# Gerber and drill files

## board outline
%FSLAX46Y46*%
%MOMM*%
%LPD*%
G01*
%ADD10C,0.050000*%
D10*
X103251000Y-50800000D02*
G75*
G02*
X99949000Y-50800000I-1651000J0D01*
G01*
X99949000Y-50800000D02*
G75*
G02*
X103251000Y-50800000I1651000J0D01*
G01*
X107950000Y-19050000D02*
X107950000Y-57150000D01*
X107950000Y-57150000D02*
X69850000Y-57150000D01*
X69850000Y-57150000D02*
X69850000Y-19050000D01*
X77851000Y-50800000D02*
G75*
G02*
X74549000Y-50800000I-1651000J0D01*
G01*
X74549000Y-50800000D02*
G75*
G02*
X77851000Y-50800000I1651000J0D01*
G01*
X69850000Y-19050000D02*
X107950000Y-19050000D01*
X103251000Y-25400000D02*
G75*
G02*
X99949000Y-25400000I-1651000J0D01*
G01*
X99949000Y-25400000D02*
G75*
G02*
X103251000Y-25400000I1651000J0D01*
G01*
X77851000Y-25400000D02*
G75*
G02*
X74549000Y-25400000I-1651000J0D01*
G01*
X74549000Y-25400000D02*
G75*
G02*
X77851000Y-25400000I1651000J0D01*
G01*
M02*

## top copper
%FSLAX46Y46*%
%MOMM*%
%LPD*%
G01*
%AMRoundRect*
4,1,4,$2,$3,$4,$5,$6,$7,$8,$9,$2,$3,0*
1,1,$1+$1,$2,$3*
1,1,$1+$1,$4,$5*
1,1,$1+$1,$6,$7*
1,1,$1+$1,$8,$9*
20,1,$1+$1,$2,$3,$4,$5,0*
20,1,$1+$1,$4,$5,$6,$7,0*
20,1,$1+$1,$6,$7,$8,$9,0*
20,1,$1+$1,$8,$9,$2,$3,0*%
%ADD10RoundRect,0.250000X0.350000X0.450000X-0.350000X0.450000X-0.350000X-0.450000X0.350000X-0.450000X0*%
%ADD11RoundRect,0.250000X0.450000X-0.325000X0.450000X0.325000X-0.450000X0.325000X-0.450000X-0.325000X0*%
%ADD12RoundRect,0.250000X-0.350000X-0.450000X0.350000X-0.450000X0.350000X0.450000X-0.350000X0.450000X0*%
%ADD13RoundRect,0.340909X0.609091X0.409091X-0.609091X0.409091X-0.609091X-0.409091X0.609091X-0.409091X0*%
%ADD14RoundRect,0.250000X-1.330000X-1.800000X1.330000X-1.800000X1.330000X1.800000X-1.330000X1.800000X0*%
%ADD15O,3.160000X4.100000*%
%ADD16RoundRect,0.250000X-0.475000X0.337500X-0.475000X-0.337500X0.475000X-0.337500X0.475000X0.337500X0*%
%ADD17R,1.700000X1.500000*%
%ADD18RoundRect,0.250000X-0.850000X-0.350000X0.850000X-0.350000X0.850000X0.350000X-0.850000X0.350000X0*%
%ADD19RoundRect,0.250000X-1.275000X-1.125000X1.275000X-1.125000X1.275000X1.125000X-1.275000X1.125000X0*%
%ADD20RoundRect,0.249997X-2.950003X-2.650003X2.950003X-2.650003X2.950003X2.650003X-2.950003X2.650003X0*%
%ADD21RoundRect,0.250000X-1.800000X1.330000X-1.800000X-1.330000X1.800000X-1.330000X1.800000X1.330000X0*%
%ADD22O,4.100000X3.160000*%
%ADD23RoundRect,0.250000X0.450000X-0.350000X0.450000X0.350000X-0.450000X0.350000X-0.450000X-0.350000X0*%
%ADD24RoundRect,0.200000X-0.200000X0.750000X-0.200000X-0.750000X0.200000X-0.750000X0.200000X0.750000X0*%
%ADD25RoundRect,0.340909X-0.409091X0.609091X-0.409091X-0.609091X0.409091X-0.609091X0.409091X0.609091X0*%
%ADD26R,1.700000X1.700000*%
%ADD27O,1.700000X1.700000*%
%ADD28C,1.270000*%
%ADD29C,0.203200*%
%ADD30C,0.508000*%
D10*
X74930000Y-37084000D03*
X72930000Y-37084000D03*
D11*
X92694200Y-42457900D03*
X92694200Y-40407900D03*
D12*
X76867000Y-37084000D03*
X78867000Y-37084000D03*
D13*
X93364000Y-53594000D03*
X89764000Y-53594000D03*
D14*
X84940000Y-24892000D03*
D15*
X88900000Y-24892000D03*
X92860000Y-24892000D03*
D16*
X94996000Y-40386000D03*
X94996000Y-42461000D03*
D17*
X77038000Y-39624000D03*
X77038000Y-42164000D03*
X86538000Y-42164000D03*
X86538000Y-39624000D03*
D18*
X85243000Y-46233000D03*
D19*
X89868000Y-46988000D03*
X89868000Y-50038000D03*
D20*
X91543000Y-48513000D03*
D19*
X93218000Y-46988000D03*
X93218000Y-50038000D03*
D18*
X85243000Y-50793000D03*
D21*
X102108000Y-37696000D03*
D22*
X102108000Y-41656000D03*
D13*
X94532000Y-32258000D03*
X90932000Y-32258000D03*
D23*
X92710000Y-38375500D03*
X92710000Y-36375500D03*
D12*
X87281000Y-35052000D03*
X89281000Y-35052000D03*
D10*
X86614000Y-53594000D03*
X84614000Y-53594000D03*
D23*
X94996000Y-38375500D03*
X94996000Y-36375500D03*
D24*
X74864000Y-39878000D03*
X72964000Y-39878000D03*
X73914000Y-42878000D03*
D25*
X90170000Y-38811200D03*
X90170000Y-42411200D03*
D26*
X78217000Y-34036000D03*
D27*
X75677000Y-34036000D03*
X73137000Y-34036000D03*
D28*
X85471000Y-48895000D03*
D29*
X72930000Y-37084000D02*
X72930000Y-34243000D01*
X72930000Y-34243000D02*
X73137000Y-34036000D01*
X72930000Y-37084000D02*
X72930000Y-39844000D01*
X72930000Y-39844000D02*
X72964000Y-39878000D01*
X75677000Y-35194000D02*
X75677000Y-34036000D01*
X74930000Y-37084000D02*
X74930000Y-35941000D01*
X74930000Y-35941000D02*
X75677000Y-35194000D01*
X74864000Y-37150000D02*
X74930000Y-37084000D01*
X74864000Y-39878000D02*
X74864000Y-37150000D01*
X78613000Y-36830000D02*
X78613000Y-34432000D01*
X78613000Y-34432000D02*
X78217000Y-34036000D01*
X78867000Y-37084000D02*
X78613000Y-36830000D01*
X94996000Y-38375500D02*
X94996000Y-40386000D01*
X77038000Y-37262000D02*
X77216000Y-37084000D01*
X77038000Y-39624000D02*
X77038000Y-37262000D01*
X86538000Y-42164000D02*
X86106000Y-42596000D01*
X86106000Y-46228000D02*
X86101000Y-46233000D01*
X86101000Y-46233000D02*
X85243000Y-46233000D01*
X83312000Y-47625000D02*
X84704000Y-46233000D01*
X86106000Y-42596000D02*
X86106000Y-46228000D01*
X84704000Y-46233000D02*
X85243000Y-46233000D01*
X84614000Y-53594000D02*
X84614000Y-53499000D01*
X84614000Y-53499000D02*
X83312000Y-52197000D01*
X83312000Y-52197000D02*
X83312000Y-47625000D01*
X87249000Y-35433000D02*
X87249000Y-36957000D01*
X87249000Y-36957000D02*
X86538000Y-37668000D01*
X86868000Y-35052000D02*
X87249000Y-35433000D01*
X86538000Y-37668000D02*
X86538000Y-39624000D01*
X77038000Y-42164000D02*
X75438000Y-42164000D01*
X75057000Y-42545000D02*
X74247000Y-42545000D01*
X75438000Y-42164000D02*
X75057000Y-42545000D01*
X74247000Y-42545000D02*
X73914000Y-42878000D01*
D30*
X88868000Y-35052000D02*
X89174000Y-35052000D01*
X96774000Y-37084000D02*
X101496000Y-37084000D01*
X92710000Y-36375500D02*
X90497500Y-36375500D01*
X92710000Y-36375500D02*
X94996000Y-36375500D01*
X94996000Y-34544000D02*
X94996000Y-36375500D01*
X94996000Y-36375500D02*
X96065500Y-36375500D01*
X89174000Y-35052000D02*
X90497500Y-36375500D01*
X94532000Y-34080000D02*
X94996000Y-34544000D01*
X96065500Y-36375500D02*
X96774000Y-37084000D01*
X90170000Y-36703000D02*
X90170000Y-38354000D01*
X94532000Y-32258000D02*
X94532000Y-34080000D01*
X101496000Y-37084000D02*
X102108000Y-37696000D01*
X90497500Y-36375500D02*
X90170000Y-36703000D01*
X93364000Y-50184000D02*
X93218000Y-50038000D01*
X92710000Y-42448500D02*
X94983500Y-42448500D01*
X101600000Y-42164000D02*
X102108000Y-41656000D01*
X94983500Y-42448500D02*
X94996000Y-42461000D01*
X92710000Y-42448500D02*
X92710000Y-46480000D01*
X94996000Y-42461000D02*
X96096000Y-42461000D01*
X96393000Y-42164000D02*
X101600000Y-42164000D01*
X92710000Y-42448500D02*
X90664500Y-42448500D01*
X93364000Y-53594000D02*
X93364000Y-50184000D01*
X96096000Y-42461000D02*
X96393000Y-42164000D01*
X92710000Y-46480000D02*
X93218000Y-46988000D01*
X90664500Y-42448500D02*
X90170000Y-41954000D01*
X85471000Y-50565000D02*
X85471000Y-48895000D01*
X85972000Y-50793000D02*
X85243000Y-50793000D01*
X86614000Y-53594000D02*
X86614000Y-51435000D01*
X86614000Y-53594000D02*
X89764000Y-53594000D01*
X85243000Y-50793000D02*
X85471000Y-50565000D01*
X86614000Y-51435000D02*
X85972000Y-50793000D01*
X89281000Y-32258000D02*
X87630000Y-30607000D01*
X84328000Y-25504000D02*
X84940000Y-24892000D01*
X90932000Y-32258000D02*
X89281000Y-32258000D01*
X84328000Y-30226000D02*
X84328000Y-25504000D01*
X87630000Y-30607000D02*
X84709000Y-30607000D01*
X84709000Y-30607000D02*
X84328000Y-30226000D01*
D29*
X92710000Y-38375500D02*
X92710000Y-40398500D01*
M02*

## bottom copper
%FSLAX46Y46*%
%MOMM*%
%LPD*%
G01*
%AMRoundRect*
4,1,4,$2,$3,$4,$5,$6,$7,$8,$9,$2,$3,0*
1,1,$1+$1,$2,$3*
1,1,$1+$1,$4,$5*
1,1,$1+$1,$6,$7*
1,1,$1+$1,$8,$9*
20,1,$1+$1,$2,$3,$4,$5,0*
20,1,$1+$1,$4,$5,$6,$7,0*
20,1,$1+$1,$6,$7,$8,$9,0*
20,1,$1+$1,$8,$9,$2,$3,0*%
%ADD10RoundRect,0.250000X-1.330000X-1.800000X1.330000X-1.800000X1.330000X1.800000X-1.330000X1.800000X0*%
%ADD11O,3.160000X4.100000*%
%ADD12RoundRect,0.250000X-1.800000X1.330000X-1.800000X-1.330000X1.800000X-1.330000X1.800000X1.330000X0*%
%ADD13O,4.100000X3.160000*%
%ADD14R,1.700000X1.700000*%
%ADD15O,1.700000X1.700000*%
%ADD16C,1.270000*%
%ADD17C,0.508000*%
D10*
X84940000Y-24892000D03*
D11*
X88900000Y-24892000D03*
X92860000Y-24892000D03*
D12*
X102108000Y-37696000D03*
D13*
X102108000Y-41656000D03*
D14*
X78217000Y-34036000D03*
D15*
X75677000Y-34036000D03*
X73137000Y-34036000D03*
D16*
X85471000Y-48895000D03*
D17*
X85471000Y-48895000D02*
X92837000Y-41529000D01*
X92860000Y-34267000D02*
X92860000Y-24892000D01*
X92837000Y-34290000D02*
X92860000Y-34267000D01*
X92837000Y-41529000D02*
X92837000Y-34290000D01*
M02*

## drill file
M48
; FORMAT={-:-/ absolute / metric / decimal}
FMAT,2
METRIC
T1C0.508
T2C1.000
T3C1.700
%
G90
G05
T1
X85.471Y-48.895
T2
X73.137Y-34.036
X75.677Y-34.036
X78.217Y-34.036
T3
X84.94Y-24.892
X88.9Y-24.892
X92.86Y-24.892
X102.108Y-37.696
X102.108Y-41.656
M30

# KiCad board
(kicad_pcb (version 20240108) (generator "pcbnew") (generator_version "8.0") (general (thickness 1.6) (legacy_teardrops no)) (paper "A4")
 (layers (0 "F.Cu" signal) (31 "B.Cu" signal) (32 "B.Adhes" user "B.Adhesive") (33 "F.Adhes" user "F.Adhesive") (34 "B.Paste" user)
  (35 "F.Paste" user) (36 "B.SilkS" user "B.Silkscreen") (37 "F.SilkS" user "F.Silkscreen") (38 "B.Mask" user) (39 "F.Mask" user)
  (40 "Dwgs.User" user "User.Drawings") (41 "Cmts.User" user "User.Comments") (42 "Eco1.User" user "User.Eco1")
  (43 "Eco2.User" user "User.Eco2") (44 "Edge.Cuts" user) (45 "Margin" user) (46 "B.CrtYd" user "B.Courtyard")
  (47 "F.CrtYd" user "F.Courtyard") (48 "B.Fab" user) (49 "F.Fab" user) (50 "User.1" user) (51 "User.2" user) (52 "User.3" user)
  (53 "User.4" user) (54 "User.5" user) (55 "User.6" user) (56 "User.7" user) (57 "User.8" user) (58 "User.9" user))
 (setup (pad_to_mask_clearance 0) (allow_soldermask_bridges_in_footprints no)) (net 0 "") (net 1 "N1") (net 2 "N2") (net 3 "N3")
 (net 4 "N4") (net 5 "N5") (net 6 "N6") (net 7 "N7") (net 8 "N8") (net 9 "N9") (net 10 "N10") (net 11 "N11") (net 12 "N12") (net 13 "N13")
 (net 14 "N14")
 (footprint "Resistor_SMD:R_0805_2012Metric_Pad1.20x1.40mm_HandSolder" (layer "F.Cu") (at 73.93 37.084 180)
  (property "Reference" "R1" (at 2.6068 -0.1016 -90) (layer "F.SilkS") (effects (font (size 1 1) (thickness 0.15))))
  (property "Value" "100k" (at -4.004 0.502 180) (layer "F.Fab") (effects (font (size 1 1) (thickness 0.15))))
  (pad "1" smd roundrect (at -1 0 180) (size 1.2 1.4) (layers "F.Cu" "F.Paste" "F.Mask") (roundrect_rratio 0.208333) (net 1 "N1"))
  (pad "2" smd roundrect (at 1 0 180) (size 1.2 1.4) (layers "F.Cu" "F.Paste" "F.Mask") (roundrect_rratio 0.208333) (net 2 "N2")))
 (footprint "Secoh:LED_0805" (layer "F.Cu") (at 92.71 41.4235 90)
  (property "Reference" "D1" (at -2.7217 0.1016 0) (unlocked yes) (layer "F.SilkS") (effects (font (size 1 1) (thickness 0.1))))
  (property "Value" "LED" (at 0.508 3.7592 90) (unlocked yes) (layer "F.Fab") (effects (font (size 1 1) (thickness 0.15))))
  (pad "1" smd roundrect (at -1.0344 -0.0158 90) (size 1.15 1.4) (layers "F.Cu" "F.Paste" "F.Mask") (roundrect_rratio 0.217391) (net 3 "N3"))
  (pad "2" smd roundrect (at 1.0156 -0.0158 90) (size 1.15 1.4) (layers "F.Cu" "F.Paste" "F.Mask") (roundrect_rratio 0.217391) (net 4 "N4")))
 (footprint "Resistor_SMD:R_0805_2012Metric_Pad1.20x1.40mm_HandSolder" (layer "F.Cu") (at 77.867 37.084)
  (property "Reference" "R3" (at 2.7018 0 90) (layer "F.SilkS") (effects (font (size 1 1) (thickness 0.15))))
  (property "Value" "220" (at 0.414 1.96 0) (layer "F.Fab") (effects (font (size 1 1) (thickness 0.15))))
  (pad "1" smd roundrect (at -1 0) (size 1.2 1.4) (layers "F.Cu" "F.Paste" "F.Mask") (roundrect_rratio 0.208333) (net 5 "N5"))
  (pad "2" smd roundrect (at 1 0) (size 1.2 1.4) (layers "F.Cu" "F.Paste" "F.Mask") (roundrect_rratio 0.208333) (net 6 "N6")))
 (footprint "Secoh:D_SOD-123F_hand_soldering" (layer "F.Cu") (at 91.564 53.594 180)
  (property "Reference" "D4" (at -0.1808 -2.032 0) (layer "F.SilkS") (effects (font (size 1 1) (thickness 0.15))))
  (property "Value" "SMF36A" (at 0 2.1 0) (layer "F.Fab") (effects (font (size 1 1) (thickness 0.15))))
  (pad "1" smd roundrect (at -1.8 0 180) (size 1.9 1.5) (layers "F.Cu" "F.Paste" "F.Mask") (roundrect_rratio 0.2272727273) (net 3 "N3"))
  (pad "2" smd roundrect (at 1.8 0 180) (size 1.9 1.5) (layers "F.Cu" "F.Paste" "F.Mask") (roundrect_rratio 0.2272727273) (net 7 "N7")))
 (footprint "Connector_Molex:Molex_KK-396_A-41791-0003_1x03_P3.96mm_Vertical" (layer "F.Cu") (at 84.94 24.892)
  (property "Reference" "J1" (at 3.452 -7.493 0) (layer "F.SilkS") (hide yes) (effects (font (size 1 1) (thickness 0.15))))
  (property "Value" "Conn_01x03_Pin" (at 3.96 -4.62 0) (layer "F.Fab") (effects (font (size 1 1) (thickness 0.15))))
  (pad "1" thru_hole roundrect (at 0 0) (size 3.16 4.1) (drill 1.7) (layers "*.Cu" "*.Mask") (remove_unused_layers no)
   (roundrect_rratio 0.079114) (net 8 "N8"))
  (pad "2" thru_hole oval (at 3.96 0) (size 3.16 4.1) (drill 1.7) (layers "*.Cu" "*.Mask") (remove_unused_layers no) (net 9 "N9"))
  (pad "3" thru_hole oval (at 7.92 0) (size 3.16 4.1) (drill 1.7) (layers "*.Cu" "*.Mask") (remove_unused_layers no) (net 7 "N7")))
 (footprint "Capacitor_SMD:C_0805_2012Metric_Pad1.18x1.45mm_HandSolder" (layer "F.Cu") (at 94.996 41.4235 -90)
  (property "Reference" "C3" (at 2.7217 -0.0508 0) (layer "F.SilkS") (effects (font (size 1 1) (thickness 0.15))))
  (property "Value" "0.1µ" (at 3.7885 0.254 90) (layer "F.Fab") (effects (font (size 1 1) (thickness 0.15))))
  (pad "1" smd roundrect (at -1.0375 0 270) (size 1.175 1.45) (layers "F.Cu" "F.Paste" "F.Mask") (roundrect_rratio 0.212766) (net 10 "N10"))
  (pad "2" smd roundrect (at 1.0375 0 270) (size 1.175 1.45) (layers "F.Cu" "F.Paste" "F.Mask") (roundrect_rratio 0.212766) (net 3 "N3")))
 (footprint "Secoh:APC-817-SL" (layer "F.Cu") (at 81.788 40.894 -90)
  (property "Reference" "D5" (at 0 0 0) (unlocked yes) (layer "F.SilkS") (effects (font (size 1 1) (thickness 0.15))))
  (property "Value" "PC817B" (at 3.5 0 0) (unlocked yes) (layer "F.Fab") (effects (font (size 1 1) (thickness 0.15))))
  (pad "1" smd rect (at -1.27 4.75 270) (size 1.5 1.7) (layers "F.Cu" "F.Paste" "F.Mask") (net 5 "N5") (thermal_bridge_angle 45))
  (pad "2" smd rect (at 1.27 4.75 270) (size 1.5 1.7) (layers "F.Cu" "F.Paste" "F.Mask") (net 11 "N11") (thermal_bridge_angle 45))
  (pad "3" smd rect (at 1.27 -4.75 270) (size 1.5 1.7) (layers "F.Cu" "F.Paste" "F.Mask") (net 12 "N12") (thermal_bridge_angle 45))
  (pad "4" smd rect (at -1.27 -4.75 270) (size 1.5 1.7) (layers "F.Cu" "F.Paste" "F.Mask") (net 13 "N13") (thermal_bridge_angle 45)))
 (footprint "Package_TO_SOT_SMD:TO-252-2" (layer "F.Cu") (at 90.283 48.513)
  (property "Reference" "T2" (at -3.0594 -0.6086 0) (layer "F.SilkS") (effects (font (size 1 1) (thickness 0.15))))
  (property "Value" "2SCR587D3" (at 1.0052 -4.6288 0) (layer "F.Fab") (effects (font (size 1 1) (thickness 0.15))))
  (pad "1" smd roundrect (at -5.04 -2.28) (size 2.2 1.2) (layers "F.Cu" "F.Paste" "F.Mask") (roundrect_rratio 0.208333) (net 12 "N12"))
  (pad "2" smd roundrect (at -0.415 -1.525) (size 3.05 2.75) (layers "F.Cu" "F.Paste") (roundrect_rratio 0.090909) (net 3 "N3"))
  (pad "2" smd roundrect (at -0.415 1.525) (size 3.05 2.75) (layers "F.Cu" "F.Paste") (roundrect_rratio 0.090909) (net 3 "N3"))
  (pad "2" smd roundrect (at 1.26 0) (size 6.4 5.8) (layers "F.Cu" "F.Mask") (roundrect_rratio 0.043103) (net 3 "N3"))
  (pad "2" smd roundrect (at 2.935 -1.525) (size 3.05 2.75) (layers "F.Cu" "F.Paste") (roundrect_rratio 0.090909) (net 3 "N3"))
  (pad "2" smd roundrect (at 2.935 1.525) (size 3.05 2.75) (layers "F.Cu" "F.Paste") (roundrect_rratio 0.090909) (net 3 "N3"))
  (pad "3" smd roundrect (at -5.04 2.28) (size 2.2 1.2) (layers "F.Cu" "F.Paste" "F.Mask") (roundrect_rratio 0.208333) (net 7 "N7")))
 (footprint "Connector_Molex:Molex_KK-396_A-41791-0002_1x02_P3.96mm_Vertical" (layer "F.Cu") (at 102.108 37.696 -90)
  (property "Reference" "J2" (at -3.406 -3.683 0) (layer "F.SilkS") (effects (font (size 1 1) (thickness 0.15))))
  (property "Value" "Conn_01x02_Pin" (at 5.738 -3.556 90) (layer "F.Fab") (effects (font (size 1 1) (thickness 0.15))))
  (pad "1" thru_hole roundrect (at 0 0 270) (size 3.16 4.1) (drill 1.7) (layers "*.Cu" "*.Mask") (remove_unused_layers no)
   (roundrect_rratio 0.079114) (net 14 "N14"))
  (pad "2" thru_hole oval (at 3.96 0 270) (size 3.16 4.1) (drill 1.7) (layers "*.Cu" "*.Mask") (remove_unused_layers no) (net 3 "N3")))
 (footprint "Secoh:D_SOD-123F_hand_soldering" (layer "F.Cu") (at 92.732 32.258 180)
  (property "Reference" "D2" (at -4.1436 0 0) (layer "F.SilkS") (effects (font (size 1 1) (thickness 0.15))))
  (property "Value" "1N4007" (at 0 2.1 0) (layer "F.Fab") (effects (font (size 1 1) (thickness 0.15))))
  (pad "1" smd roundrect (at -1.8 0 180) (size 1.9 1.5) (layers "F.Cu" "F.Paste" "F.Mask") (roundrect_rratio 0.2272727273) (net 14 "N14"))
  (pad "2" smd roundrect (at 1.8 0 180) (size 1.9 1.5) (layers "F.Cu" "F.Paste" "F.Mask") (roundrect_rratio 0.2272727273) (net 8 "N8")))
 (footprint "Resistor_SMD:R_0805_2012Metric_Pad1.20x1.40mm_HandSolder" (layer "F.Cu") (at 92.71 37.3755 90)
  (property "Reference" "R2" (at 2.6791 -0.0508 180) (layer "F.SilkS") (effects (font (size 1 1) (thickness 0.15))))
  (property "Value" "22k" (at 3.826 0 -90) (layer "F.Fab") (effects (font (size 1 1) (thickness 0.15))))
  (pad "1" smd roundrect (at -1 0 90) (size 1.2 1.4) (layers "F.Cu" "F.Paste" "F.Mask") (roundrect_rratio 0.208333) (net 4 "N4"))
  (pad "2" smd roundrect (at 1 0 90) (size 1.2 1.4) (layers "F.Cu" "F.Paste" "F.Mask") (roundrect_rratio 0.208333) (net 14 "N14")))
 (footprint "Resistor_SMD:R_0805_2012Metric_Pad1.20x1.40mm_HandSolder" (layer "F.Cu") (at 88.281 35.052)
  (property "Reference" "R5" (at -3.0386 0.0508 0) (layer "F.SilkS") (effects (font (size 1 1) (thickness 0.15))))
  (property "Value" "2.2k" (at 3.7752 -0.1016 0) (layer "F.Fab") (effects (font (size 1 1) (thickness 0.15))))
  (pad "1" smd roundrect (at -1 0) (size 1.2 1.4) (layers "F.Cu" "F.Paste" "F.Mask") (roundrect_rratio 0.208333) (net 13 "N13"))
  (pad "2" smd roundrect (at 1 0) (size 1.2 1.4) (layers "F.Cu" "F.Paste" "F.Mask") (roundrect_rratio 0.208333) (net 14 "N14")))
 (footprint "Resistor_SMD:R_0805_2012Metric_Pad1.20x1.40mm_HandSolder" (layer "F.Cu") (at 85.614 53.594 180)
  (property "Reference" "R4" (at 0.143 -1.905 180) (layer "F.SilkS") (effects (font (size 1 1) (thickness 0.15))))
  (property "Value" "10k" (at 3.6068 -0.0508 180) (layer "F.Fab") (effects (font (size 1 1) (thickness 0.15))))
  (pad "1" smd roundrect (at -1 0 180) (size 1.2 1.4) (layers "F.Cu" "F.Paste" "F.Mask") (roundrect_rratio 0.208333) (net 7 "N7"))
  (pad "2" smd roundrect (at 1 0 180) (size 1.2 1.4) (layers "F.Cu" "F.Paste" "F.Mask") (roundrect_rratio 0.208333) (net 12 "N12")))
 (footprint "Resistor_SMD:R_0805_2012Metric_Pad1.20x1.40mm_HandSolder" (layer "F.Cu") (at 94.996 37.3755 90)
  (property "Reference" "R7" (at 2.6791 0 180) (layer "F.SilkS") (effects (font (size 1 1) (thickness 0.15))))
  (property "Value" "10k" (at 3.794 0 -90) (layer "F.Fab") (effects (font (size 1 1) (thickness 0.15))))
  (pad "1" smd roundrect (at -1 0 90) (size 1.2 1.4) (layers "F.Cu" "F.Paste" "F.Mask") (roundrect_rratio 0.208333) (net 10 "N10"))
  (pad "2" smd roundrect (at 1 0 90) (size 1.2 1.4) (layers "F.Cu" "F.Paste" "F.Mask") (roundrect_rratio 0.208333) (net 14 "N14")))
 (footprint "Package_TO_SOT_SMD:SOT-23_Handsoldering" (layer "F.Cu") (at 73.914 41.378 -90)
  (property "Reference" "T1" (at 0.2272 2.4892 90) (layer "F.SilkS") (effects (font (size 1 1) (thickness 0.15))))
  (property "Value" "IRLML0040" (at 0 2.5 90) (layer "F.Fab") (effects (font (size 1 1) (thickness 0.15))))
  (pad "1" smd roundrect (at -1.5 -0.95 270) (size 1.9 0.8) (layers "F.Cu" "F.Paste" "F.Mask") (roundrect_rratio 0.25) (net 1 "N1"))
  (pad "2" smd roundrect (at -1.5 0.95 270) (size 1.9 0.8) (layers "F.Cu" "F.Paste" "F.Mask") (roundrect_rratio 0.25) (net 2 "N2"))
  (pad "3" smd roundrect (at 1.5 0 270) (size 1.9 0.8) (layers "F.Cu" "F.Paste" "F.Mask") (roundrect_rratio 0.25) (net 11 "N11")))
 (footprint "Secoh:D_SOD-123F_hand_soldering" (layer "F.Cu") (at 90.17 40.6112 -90)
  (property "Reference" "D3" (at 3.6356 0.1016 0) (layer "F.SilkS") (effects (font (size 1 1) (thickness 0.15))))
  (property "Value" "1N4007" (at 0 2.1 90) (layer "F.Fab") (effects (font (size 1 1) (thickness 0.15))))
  (pad "1" smd roundrect (at -1.8 0 270) (size 1.9 1.5) (layers "F.Cu" "F.Paste" "F.Mask") (roundrect_rratio 0.2272727273) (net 14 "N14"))
  (pad "2" smd roundrect (at 1.8 0 270) (size 1.9 1.5) (layers "F.Cu" "F.Paste" "F.Mask") (roundrect_rratio 0.2272727273) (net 3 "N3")))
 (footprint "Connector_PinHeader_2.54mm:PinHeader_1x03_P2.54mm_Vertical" (layer "F.Cu") (at 78.217 34.036 -90)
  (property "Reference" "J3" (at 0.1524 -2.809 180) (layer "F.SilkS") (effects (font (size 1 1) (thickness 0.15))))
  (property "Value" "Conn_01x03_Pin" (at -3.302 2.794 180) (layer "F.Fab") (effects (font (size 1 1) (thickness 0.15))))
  (pad "1" thru_hole rect (at 0 0 270) (size 1.7 1.7) (drill 1) (layers "*.Cu" "*.Mask") (remove_unused_layers no) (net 6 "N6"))
  (pad "2" thru_hole oval (at 0 2.54 270) (size 1.7 1.7) (drill 1) (layers "*.Cu" "*.Mask") (remove_unused_layers no) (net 1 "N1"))
  (pad "3" thru_hole oval (at 0 5.08 270) (size 1.7 1.7) (drill 1) (layers "*.Cu" "*.Mask") (remove_unused_layers no) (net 2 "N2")))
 (gr_circle (center 101.6 50.8) (end 103.251 50.8) (stroke (width 0.05) (type default)) (fill none) (layer "Edge.Cuts"))
 (gr_line (start 107.95 19.05) (end 107.95 57.15) (stroke (width 0.05) (type default)) (layer "Edge.Cuts"))
 (gr_line (start 107.95 57.15) (end 69.85 57.15) (stroke (width 0.05) (type default)) (layer "Edge.Cuts"))
 (gr_line (start 69.85 57.15) (end 69.85 19.05) (stroke (width 0.05) (type default)) (layer "Edge.Cuts"))
 (gr_circle (center 76.2 50.8) (end 77.851 50.8) (stroke (width 0.05) (type solid)) (fill none) (layer "Edge.Cuts"))
 (gr_line (start 69.85 19.05) (end 107.95 19.05) (stroke (width 0.05) (type default)) (layer "Edge.Cuts"))
 (gr_circle (center 101.6 25.4) (end 103.251 25.4) (stroke (width 0.05) (type solid)) (fill none) (layer "Edge.Cuts"))
 (gr_circle (center 76.2 25.4) (end 77.851 25.4) (stroke (width 0.05) (type solid)) (fill none) (layer "Edge.Cuts"))
 (segment (start 72.93 37.084) (end 72.93 34.243) (width 0.2032) (layer "F.Cu") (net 2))
 (segment (start 72.93 34.243) (end 73.137 34.036) (width 0.2032) (layer "F.Cu") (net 2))
 (segment (start 72.93 37.084) (end 72.93 39.844) (width 0.2032) (layer "F.Cu") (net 2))
 (segment (start 72.93 39.844) (end 72.964 39.878) (width 0.2032) (layer "F.Cu") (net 2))
 (segment (start 75.677 35.194) (end 75.677 34.036) (width 0.2032) (layer "F.Cu") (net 1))
 (segment (start 74.93 37.084) (end 74.93 35.941) (width 0.2032) (layer "F.Cu") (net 1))
 (segment (start 74.93 35.941) (end 75.677 35.194) (width 0.2032) (layer "F.Cu") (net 1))
 (segment (start 74.864 37.15) (end 74.93 37.084) (width 0.2032) (layer "F.Cu") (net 1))
 (segment (start 74.864 39.878) (end 74.864 37.15) (width 0.2032) (layer "F.Cu") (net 1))
 (segment (start 78.613 36.83) (end 78.613 34.432) (width 0.2032) (layer "F.Cu") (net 6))
 (segment (start 78.613 34.432) (end 78.217 34.036) (width 0.2032) (layer "F.Cu") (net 6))
 (segment (start 78.867 37.084) (end 78.613 36.83) (width 0.2032) (layer "F.Cu") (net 6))
 (segment (start 94.996 38.3755) (end 94.996 40.386) (width 0.2032) (layer "F.Cu") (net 10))
 (segment (start 77.038 37.262) (end 77.216 37.084) (width 0.2032) (layer "F.Cu") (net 5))
 (segment (start 77.038 39.624) (end 77.038 37.262) (width 0.2032) (layer "F.Cu") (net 5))
 (segment (start 86.538 42.164) (end 86.106 42.596) (width 0.2032) (layer "F.Cu") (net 12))
 (segment (start 86.106 46.228) (end 86.101 46.233) (width 0.2032) (layer "F.Cu") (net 12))
 (segment (start 86.101 46.233) (end 85.243 46.233) (width 0.2032) (layer "F.Cu") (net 12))
 (segment (start 83.312 47.625) (end 84.704 46.233) (width 0.2032) (layer "F.Cu") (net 12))
 (segment (start 86.106 42.596) (end 86.106 46.228) (width 0.2032) (layer "F.Cu") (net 12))
 (segment (start 84.704 46.233) (end 85.243 46.233) (width 0.2032) (layer "F.Cu") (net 12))
 (segment (start 84.614 53.594) (end 84.614 53.499) (width 0.2032) (layer "F.Cu") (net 12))
 (segment (start 84.614 53.499) (end 83.312 52.197) (width 0.2032) (layer "F.Cu") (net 12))
 (segment (start 83.312 52.197) (end 83.312 47.625) (width 0.2032) (layer "F.Cu") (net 12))
 (segment (start 87.249 35.433) (end 87.249 36.957) (width 0.2032) (layer "F.Cu") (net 13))
 (segment (start 87.249 36.957) (end 86.538 37.668) (width 0.2032) (layer "F.Cu") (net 13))
 (segment (start 86.868 35.052) (end 87.249 35.433) (width 0.2032) (layer "F.Cu") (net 13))
 (segment (start 86.538 37.668) (end 86.538 39.624) (width 0.2032) (layer "F.Cu") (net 13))
 (segment (start 77.038 42.164) (end 75.438 42.164) (width 0.2032) (layer "F.Cu") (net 11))
 (segment (start 75.057 42.545) (end 74.247 42.545) (width 0.2032) (layer "F.Cu") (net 11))
 (segment (start 75.438 42.164) (end 75.057 42.545) (width 0.2032) (layer "F.Cu") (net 11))
 (segment (start 74.247 42.545) (end 73.914 42.878) (width 0.2032) (layer "F.Cu") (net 11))
 (segment (start 88.868 35.052) (end 89.174 35.052) (width 0.508) (layer "F.Cu") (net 14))
 (segment (start 96.774 37.084) (end 101.496 37.084) (width 0.508) (layer "F.Cu") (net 14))
 (segment (start 92.71 36.3755) (end 90.4975 36.3755) (width 0.508) (layer "F.Cu") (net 14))
 (segment (start 92.71 36.3755) (end 94.996 36.3755) (width 0.508) (layer "F.Cu") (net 14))
 (segment (start 94.996 34.544) (end 94.996 36.3755) (width 0.508) (layer "F.Cu") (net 14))
 (segment (start 94.996 36.3755) (end 96.0655 36.3755) (width 0.508) (layer "F.Cu") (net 14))
 (segment (start 89.174 35.052) (end 90.4975 36.3755) (width 0.508) (layer "F.Cu") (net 14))
 (segment (start 94.532 34.08) (end 94.996 34.544) (width 0.508) (layer "F.Cu") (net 14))
 (segment (start 96.0655 36.3755) (end 96.774 37.084) (width 0.508) (layer "F.Cu") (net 14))
 (segment (start 90.17 36.703) (end 90.17 38.354) (width 0.508) (layer "F.Cu") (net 14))
 (segment (start 94.532 32.258) (end 94.532 34.08) (width 0.508) (layer "F.Cu") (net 14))
 (segment (start 101.496 37.084) (end 102.108 37.696) (width 0.508) (layer "F.Cu") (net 14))
 (segment (start 90.4975 36.3755) (end 90.17 36.703) (width 0.508) (layer "F.Cu") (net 14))
 (segment (start 93.364 50.184) (end 93.218 50.038) (width 0.508) (layer "F.Cu") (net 3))
 (segment (start 92.71 42.4485) (end 94.9835 42.4485) (width 0.508) (layer "F.Cu") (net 3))
 (segment (start 101.6 42.164) (end 102.108 41.656) (width 0.508) (layer "F.Cu") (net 3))
 (segment (start 94.9835 42.4485) (end 94.996 42.461) (width 0.508) (layer "F.Cu") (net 3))
 (segment (start 92.71 42.4485) (end 92.71 46.48) (width 0.508) (layer "F.Cu") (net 3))
 (segment (start 94.996 42.461) (end 96.096 42.461) (width 0.508) (layer "F.Cu") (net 3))
 (segment (start 96.393 42.164) (end 101.6 42.164) (width 0.508) (layer "F.Cu") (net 3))
 (segment (start 92.71 42.4485) (end 90.6645 42.4485) (width 0.508) (layer "F.Cu") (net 3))
 (segment (start 93.364 53.594) (end 93.364 50.184) (width 0.508) (layer "F.Cu") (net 3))
 (segment (start 96.096 42.461) (end 96.393 42.164) (width 0.508) (layer "F.Cu") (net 3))
 (segment (start 92.71 46.48) (end 93.218 46.988) (width 0.508) (layer "F.Cu") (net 3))
 (segment (start 90.6645 42.4485) (end 90.17 41.954) (width 0.508) (layer "F.Cu") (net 3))
 (segment (start 85.471 50.565) (end 85.471 48.895) (width 0.508) (layer "F.Cu") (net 7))
 (segment (start 85.972 50.793) (end 85.243 50.793) (width 0.508) (layer "F.Cu") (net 7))
 (segment (start 86.614 53.594) (end 86.614 51.435) (width 0.508) (layer "F.Cu") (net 7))
 (segment (start 86.614 53.594) (end 89.764 53.594) (width 0.508) (layer "F.Cu") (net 7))
 (segment (start 85.243 50.793) (end 85.471 50.565) (width 0.508) (layer "F.Cu") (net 7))
 (segment (start 86.614 51.435) (end 85.972 50.793) (width 0.508) (layer "F.Cu") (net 7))
 (via (at 85.471 48.895) (size 1.27) (drill 0.508) (layers "F.Cu" "B.Cu") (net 7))
 (segment (start 85.471 48.895) (end 92.837 41.529) (width 0.508) (layer "B.Cu") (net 7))
 (segment (start 92.86 34.267) (end 92.86 24.892) (width 0.508) (layer "B.Cu") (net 7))
 (segment (start 92.837 34.29) (end 92.86 34.267) (width 0.508) (layer "B.Cu") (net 7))
 (segment (start 92.837 41.529) (end 92.837 34.29) (width 0.508) (layer "B.Cu") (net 7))
 (segment (start 89.281 32.258) (end 87.63 30.607) (width 0.508) (layer "F.Cu") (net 8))
 (segment (start 84.328 25.504) (end 84.94 24.892) (width 0.508) (layer "F.Cu") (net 8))
 (segment (start 90.932 32.258) (end 89.281 32.258) (width 0.508) (layer "F.Cu") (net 8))
 (segment (start 84.328 30.226) (end 84.328 25.504) (width 0.508) (layer "F.Cu") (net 8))
 (segment (start 87.63 30.607) (end 84.709 30.607) (width 0.508) (layer "F.Cu") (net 8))
 (segment (start 84.709 30.607) (end 84.328 30.226) (width 0.508) (layer "F.Cu") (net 8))
 (segment (start 92.71 38.3755) (end 92.71 40.3985) (width 0.2032) (layer "F.Cu") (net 4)))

